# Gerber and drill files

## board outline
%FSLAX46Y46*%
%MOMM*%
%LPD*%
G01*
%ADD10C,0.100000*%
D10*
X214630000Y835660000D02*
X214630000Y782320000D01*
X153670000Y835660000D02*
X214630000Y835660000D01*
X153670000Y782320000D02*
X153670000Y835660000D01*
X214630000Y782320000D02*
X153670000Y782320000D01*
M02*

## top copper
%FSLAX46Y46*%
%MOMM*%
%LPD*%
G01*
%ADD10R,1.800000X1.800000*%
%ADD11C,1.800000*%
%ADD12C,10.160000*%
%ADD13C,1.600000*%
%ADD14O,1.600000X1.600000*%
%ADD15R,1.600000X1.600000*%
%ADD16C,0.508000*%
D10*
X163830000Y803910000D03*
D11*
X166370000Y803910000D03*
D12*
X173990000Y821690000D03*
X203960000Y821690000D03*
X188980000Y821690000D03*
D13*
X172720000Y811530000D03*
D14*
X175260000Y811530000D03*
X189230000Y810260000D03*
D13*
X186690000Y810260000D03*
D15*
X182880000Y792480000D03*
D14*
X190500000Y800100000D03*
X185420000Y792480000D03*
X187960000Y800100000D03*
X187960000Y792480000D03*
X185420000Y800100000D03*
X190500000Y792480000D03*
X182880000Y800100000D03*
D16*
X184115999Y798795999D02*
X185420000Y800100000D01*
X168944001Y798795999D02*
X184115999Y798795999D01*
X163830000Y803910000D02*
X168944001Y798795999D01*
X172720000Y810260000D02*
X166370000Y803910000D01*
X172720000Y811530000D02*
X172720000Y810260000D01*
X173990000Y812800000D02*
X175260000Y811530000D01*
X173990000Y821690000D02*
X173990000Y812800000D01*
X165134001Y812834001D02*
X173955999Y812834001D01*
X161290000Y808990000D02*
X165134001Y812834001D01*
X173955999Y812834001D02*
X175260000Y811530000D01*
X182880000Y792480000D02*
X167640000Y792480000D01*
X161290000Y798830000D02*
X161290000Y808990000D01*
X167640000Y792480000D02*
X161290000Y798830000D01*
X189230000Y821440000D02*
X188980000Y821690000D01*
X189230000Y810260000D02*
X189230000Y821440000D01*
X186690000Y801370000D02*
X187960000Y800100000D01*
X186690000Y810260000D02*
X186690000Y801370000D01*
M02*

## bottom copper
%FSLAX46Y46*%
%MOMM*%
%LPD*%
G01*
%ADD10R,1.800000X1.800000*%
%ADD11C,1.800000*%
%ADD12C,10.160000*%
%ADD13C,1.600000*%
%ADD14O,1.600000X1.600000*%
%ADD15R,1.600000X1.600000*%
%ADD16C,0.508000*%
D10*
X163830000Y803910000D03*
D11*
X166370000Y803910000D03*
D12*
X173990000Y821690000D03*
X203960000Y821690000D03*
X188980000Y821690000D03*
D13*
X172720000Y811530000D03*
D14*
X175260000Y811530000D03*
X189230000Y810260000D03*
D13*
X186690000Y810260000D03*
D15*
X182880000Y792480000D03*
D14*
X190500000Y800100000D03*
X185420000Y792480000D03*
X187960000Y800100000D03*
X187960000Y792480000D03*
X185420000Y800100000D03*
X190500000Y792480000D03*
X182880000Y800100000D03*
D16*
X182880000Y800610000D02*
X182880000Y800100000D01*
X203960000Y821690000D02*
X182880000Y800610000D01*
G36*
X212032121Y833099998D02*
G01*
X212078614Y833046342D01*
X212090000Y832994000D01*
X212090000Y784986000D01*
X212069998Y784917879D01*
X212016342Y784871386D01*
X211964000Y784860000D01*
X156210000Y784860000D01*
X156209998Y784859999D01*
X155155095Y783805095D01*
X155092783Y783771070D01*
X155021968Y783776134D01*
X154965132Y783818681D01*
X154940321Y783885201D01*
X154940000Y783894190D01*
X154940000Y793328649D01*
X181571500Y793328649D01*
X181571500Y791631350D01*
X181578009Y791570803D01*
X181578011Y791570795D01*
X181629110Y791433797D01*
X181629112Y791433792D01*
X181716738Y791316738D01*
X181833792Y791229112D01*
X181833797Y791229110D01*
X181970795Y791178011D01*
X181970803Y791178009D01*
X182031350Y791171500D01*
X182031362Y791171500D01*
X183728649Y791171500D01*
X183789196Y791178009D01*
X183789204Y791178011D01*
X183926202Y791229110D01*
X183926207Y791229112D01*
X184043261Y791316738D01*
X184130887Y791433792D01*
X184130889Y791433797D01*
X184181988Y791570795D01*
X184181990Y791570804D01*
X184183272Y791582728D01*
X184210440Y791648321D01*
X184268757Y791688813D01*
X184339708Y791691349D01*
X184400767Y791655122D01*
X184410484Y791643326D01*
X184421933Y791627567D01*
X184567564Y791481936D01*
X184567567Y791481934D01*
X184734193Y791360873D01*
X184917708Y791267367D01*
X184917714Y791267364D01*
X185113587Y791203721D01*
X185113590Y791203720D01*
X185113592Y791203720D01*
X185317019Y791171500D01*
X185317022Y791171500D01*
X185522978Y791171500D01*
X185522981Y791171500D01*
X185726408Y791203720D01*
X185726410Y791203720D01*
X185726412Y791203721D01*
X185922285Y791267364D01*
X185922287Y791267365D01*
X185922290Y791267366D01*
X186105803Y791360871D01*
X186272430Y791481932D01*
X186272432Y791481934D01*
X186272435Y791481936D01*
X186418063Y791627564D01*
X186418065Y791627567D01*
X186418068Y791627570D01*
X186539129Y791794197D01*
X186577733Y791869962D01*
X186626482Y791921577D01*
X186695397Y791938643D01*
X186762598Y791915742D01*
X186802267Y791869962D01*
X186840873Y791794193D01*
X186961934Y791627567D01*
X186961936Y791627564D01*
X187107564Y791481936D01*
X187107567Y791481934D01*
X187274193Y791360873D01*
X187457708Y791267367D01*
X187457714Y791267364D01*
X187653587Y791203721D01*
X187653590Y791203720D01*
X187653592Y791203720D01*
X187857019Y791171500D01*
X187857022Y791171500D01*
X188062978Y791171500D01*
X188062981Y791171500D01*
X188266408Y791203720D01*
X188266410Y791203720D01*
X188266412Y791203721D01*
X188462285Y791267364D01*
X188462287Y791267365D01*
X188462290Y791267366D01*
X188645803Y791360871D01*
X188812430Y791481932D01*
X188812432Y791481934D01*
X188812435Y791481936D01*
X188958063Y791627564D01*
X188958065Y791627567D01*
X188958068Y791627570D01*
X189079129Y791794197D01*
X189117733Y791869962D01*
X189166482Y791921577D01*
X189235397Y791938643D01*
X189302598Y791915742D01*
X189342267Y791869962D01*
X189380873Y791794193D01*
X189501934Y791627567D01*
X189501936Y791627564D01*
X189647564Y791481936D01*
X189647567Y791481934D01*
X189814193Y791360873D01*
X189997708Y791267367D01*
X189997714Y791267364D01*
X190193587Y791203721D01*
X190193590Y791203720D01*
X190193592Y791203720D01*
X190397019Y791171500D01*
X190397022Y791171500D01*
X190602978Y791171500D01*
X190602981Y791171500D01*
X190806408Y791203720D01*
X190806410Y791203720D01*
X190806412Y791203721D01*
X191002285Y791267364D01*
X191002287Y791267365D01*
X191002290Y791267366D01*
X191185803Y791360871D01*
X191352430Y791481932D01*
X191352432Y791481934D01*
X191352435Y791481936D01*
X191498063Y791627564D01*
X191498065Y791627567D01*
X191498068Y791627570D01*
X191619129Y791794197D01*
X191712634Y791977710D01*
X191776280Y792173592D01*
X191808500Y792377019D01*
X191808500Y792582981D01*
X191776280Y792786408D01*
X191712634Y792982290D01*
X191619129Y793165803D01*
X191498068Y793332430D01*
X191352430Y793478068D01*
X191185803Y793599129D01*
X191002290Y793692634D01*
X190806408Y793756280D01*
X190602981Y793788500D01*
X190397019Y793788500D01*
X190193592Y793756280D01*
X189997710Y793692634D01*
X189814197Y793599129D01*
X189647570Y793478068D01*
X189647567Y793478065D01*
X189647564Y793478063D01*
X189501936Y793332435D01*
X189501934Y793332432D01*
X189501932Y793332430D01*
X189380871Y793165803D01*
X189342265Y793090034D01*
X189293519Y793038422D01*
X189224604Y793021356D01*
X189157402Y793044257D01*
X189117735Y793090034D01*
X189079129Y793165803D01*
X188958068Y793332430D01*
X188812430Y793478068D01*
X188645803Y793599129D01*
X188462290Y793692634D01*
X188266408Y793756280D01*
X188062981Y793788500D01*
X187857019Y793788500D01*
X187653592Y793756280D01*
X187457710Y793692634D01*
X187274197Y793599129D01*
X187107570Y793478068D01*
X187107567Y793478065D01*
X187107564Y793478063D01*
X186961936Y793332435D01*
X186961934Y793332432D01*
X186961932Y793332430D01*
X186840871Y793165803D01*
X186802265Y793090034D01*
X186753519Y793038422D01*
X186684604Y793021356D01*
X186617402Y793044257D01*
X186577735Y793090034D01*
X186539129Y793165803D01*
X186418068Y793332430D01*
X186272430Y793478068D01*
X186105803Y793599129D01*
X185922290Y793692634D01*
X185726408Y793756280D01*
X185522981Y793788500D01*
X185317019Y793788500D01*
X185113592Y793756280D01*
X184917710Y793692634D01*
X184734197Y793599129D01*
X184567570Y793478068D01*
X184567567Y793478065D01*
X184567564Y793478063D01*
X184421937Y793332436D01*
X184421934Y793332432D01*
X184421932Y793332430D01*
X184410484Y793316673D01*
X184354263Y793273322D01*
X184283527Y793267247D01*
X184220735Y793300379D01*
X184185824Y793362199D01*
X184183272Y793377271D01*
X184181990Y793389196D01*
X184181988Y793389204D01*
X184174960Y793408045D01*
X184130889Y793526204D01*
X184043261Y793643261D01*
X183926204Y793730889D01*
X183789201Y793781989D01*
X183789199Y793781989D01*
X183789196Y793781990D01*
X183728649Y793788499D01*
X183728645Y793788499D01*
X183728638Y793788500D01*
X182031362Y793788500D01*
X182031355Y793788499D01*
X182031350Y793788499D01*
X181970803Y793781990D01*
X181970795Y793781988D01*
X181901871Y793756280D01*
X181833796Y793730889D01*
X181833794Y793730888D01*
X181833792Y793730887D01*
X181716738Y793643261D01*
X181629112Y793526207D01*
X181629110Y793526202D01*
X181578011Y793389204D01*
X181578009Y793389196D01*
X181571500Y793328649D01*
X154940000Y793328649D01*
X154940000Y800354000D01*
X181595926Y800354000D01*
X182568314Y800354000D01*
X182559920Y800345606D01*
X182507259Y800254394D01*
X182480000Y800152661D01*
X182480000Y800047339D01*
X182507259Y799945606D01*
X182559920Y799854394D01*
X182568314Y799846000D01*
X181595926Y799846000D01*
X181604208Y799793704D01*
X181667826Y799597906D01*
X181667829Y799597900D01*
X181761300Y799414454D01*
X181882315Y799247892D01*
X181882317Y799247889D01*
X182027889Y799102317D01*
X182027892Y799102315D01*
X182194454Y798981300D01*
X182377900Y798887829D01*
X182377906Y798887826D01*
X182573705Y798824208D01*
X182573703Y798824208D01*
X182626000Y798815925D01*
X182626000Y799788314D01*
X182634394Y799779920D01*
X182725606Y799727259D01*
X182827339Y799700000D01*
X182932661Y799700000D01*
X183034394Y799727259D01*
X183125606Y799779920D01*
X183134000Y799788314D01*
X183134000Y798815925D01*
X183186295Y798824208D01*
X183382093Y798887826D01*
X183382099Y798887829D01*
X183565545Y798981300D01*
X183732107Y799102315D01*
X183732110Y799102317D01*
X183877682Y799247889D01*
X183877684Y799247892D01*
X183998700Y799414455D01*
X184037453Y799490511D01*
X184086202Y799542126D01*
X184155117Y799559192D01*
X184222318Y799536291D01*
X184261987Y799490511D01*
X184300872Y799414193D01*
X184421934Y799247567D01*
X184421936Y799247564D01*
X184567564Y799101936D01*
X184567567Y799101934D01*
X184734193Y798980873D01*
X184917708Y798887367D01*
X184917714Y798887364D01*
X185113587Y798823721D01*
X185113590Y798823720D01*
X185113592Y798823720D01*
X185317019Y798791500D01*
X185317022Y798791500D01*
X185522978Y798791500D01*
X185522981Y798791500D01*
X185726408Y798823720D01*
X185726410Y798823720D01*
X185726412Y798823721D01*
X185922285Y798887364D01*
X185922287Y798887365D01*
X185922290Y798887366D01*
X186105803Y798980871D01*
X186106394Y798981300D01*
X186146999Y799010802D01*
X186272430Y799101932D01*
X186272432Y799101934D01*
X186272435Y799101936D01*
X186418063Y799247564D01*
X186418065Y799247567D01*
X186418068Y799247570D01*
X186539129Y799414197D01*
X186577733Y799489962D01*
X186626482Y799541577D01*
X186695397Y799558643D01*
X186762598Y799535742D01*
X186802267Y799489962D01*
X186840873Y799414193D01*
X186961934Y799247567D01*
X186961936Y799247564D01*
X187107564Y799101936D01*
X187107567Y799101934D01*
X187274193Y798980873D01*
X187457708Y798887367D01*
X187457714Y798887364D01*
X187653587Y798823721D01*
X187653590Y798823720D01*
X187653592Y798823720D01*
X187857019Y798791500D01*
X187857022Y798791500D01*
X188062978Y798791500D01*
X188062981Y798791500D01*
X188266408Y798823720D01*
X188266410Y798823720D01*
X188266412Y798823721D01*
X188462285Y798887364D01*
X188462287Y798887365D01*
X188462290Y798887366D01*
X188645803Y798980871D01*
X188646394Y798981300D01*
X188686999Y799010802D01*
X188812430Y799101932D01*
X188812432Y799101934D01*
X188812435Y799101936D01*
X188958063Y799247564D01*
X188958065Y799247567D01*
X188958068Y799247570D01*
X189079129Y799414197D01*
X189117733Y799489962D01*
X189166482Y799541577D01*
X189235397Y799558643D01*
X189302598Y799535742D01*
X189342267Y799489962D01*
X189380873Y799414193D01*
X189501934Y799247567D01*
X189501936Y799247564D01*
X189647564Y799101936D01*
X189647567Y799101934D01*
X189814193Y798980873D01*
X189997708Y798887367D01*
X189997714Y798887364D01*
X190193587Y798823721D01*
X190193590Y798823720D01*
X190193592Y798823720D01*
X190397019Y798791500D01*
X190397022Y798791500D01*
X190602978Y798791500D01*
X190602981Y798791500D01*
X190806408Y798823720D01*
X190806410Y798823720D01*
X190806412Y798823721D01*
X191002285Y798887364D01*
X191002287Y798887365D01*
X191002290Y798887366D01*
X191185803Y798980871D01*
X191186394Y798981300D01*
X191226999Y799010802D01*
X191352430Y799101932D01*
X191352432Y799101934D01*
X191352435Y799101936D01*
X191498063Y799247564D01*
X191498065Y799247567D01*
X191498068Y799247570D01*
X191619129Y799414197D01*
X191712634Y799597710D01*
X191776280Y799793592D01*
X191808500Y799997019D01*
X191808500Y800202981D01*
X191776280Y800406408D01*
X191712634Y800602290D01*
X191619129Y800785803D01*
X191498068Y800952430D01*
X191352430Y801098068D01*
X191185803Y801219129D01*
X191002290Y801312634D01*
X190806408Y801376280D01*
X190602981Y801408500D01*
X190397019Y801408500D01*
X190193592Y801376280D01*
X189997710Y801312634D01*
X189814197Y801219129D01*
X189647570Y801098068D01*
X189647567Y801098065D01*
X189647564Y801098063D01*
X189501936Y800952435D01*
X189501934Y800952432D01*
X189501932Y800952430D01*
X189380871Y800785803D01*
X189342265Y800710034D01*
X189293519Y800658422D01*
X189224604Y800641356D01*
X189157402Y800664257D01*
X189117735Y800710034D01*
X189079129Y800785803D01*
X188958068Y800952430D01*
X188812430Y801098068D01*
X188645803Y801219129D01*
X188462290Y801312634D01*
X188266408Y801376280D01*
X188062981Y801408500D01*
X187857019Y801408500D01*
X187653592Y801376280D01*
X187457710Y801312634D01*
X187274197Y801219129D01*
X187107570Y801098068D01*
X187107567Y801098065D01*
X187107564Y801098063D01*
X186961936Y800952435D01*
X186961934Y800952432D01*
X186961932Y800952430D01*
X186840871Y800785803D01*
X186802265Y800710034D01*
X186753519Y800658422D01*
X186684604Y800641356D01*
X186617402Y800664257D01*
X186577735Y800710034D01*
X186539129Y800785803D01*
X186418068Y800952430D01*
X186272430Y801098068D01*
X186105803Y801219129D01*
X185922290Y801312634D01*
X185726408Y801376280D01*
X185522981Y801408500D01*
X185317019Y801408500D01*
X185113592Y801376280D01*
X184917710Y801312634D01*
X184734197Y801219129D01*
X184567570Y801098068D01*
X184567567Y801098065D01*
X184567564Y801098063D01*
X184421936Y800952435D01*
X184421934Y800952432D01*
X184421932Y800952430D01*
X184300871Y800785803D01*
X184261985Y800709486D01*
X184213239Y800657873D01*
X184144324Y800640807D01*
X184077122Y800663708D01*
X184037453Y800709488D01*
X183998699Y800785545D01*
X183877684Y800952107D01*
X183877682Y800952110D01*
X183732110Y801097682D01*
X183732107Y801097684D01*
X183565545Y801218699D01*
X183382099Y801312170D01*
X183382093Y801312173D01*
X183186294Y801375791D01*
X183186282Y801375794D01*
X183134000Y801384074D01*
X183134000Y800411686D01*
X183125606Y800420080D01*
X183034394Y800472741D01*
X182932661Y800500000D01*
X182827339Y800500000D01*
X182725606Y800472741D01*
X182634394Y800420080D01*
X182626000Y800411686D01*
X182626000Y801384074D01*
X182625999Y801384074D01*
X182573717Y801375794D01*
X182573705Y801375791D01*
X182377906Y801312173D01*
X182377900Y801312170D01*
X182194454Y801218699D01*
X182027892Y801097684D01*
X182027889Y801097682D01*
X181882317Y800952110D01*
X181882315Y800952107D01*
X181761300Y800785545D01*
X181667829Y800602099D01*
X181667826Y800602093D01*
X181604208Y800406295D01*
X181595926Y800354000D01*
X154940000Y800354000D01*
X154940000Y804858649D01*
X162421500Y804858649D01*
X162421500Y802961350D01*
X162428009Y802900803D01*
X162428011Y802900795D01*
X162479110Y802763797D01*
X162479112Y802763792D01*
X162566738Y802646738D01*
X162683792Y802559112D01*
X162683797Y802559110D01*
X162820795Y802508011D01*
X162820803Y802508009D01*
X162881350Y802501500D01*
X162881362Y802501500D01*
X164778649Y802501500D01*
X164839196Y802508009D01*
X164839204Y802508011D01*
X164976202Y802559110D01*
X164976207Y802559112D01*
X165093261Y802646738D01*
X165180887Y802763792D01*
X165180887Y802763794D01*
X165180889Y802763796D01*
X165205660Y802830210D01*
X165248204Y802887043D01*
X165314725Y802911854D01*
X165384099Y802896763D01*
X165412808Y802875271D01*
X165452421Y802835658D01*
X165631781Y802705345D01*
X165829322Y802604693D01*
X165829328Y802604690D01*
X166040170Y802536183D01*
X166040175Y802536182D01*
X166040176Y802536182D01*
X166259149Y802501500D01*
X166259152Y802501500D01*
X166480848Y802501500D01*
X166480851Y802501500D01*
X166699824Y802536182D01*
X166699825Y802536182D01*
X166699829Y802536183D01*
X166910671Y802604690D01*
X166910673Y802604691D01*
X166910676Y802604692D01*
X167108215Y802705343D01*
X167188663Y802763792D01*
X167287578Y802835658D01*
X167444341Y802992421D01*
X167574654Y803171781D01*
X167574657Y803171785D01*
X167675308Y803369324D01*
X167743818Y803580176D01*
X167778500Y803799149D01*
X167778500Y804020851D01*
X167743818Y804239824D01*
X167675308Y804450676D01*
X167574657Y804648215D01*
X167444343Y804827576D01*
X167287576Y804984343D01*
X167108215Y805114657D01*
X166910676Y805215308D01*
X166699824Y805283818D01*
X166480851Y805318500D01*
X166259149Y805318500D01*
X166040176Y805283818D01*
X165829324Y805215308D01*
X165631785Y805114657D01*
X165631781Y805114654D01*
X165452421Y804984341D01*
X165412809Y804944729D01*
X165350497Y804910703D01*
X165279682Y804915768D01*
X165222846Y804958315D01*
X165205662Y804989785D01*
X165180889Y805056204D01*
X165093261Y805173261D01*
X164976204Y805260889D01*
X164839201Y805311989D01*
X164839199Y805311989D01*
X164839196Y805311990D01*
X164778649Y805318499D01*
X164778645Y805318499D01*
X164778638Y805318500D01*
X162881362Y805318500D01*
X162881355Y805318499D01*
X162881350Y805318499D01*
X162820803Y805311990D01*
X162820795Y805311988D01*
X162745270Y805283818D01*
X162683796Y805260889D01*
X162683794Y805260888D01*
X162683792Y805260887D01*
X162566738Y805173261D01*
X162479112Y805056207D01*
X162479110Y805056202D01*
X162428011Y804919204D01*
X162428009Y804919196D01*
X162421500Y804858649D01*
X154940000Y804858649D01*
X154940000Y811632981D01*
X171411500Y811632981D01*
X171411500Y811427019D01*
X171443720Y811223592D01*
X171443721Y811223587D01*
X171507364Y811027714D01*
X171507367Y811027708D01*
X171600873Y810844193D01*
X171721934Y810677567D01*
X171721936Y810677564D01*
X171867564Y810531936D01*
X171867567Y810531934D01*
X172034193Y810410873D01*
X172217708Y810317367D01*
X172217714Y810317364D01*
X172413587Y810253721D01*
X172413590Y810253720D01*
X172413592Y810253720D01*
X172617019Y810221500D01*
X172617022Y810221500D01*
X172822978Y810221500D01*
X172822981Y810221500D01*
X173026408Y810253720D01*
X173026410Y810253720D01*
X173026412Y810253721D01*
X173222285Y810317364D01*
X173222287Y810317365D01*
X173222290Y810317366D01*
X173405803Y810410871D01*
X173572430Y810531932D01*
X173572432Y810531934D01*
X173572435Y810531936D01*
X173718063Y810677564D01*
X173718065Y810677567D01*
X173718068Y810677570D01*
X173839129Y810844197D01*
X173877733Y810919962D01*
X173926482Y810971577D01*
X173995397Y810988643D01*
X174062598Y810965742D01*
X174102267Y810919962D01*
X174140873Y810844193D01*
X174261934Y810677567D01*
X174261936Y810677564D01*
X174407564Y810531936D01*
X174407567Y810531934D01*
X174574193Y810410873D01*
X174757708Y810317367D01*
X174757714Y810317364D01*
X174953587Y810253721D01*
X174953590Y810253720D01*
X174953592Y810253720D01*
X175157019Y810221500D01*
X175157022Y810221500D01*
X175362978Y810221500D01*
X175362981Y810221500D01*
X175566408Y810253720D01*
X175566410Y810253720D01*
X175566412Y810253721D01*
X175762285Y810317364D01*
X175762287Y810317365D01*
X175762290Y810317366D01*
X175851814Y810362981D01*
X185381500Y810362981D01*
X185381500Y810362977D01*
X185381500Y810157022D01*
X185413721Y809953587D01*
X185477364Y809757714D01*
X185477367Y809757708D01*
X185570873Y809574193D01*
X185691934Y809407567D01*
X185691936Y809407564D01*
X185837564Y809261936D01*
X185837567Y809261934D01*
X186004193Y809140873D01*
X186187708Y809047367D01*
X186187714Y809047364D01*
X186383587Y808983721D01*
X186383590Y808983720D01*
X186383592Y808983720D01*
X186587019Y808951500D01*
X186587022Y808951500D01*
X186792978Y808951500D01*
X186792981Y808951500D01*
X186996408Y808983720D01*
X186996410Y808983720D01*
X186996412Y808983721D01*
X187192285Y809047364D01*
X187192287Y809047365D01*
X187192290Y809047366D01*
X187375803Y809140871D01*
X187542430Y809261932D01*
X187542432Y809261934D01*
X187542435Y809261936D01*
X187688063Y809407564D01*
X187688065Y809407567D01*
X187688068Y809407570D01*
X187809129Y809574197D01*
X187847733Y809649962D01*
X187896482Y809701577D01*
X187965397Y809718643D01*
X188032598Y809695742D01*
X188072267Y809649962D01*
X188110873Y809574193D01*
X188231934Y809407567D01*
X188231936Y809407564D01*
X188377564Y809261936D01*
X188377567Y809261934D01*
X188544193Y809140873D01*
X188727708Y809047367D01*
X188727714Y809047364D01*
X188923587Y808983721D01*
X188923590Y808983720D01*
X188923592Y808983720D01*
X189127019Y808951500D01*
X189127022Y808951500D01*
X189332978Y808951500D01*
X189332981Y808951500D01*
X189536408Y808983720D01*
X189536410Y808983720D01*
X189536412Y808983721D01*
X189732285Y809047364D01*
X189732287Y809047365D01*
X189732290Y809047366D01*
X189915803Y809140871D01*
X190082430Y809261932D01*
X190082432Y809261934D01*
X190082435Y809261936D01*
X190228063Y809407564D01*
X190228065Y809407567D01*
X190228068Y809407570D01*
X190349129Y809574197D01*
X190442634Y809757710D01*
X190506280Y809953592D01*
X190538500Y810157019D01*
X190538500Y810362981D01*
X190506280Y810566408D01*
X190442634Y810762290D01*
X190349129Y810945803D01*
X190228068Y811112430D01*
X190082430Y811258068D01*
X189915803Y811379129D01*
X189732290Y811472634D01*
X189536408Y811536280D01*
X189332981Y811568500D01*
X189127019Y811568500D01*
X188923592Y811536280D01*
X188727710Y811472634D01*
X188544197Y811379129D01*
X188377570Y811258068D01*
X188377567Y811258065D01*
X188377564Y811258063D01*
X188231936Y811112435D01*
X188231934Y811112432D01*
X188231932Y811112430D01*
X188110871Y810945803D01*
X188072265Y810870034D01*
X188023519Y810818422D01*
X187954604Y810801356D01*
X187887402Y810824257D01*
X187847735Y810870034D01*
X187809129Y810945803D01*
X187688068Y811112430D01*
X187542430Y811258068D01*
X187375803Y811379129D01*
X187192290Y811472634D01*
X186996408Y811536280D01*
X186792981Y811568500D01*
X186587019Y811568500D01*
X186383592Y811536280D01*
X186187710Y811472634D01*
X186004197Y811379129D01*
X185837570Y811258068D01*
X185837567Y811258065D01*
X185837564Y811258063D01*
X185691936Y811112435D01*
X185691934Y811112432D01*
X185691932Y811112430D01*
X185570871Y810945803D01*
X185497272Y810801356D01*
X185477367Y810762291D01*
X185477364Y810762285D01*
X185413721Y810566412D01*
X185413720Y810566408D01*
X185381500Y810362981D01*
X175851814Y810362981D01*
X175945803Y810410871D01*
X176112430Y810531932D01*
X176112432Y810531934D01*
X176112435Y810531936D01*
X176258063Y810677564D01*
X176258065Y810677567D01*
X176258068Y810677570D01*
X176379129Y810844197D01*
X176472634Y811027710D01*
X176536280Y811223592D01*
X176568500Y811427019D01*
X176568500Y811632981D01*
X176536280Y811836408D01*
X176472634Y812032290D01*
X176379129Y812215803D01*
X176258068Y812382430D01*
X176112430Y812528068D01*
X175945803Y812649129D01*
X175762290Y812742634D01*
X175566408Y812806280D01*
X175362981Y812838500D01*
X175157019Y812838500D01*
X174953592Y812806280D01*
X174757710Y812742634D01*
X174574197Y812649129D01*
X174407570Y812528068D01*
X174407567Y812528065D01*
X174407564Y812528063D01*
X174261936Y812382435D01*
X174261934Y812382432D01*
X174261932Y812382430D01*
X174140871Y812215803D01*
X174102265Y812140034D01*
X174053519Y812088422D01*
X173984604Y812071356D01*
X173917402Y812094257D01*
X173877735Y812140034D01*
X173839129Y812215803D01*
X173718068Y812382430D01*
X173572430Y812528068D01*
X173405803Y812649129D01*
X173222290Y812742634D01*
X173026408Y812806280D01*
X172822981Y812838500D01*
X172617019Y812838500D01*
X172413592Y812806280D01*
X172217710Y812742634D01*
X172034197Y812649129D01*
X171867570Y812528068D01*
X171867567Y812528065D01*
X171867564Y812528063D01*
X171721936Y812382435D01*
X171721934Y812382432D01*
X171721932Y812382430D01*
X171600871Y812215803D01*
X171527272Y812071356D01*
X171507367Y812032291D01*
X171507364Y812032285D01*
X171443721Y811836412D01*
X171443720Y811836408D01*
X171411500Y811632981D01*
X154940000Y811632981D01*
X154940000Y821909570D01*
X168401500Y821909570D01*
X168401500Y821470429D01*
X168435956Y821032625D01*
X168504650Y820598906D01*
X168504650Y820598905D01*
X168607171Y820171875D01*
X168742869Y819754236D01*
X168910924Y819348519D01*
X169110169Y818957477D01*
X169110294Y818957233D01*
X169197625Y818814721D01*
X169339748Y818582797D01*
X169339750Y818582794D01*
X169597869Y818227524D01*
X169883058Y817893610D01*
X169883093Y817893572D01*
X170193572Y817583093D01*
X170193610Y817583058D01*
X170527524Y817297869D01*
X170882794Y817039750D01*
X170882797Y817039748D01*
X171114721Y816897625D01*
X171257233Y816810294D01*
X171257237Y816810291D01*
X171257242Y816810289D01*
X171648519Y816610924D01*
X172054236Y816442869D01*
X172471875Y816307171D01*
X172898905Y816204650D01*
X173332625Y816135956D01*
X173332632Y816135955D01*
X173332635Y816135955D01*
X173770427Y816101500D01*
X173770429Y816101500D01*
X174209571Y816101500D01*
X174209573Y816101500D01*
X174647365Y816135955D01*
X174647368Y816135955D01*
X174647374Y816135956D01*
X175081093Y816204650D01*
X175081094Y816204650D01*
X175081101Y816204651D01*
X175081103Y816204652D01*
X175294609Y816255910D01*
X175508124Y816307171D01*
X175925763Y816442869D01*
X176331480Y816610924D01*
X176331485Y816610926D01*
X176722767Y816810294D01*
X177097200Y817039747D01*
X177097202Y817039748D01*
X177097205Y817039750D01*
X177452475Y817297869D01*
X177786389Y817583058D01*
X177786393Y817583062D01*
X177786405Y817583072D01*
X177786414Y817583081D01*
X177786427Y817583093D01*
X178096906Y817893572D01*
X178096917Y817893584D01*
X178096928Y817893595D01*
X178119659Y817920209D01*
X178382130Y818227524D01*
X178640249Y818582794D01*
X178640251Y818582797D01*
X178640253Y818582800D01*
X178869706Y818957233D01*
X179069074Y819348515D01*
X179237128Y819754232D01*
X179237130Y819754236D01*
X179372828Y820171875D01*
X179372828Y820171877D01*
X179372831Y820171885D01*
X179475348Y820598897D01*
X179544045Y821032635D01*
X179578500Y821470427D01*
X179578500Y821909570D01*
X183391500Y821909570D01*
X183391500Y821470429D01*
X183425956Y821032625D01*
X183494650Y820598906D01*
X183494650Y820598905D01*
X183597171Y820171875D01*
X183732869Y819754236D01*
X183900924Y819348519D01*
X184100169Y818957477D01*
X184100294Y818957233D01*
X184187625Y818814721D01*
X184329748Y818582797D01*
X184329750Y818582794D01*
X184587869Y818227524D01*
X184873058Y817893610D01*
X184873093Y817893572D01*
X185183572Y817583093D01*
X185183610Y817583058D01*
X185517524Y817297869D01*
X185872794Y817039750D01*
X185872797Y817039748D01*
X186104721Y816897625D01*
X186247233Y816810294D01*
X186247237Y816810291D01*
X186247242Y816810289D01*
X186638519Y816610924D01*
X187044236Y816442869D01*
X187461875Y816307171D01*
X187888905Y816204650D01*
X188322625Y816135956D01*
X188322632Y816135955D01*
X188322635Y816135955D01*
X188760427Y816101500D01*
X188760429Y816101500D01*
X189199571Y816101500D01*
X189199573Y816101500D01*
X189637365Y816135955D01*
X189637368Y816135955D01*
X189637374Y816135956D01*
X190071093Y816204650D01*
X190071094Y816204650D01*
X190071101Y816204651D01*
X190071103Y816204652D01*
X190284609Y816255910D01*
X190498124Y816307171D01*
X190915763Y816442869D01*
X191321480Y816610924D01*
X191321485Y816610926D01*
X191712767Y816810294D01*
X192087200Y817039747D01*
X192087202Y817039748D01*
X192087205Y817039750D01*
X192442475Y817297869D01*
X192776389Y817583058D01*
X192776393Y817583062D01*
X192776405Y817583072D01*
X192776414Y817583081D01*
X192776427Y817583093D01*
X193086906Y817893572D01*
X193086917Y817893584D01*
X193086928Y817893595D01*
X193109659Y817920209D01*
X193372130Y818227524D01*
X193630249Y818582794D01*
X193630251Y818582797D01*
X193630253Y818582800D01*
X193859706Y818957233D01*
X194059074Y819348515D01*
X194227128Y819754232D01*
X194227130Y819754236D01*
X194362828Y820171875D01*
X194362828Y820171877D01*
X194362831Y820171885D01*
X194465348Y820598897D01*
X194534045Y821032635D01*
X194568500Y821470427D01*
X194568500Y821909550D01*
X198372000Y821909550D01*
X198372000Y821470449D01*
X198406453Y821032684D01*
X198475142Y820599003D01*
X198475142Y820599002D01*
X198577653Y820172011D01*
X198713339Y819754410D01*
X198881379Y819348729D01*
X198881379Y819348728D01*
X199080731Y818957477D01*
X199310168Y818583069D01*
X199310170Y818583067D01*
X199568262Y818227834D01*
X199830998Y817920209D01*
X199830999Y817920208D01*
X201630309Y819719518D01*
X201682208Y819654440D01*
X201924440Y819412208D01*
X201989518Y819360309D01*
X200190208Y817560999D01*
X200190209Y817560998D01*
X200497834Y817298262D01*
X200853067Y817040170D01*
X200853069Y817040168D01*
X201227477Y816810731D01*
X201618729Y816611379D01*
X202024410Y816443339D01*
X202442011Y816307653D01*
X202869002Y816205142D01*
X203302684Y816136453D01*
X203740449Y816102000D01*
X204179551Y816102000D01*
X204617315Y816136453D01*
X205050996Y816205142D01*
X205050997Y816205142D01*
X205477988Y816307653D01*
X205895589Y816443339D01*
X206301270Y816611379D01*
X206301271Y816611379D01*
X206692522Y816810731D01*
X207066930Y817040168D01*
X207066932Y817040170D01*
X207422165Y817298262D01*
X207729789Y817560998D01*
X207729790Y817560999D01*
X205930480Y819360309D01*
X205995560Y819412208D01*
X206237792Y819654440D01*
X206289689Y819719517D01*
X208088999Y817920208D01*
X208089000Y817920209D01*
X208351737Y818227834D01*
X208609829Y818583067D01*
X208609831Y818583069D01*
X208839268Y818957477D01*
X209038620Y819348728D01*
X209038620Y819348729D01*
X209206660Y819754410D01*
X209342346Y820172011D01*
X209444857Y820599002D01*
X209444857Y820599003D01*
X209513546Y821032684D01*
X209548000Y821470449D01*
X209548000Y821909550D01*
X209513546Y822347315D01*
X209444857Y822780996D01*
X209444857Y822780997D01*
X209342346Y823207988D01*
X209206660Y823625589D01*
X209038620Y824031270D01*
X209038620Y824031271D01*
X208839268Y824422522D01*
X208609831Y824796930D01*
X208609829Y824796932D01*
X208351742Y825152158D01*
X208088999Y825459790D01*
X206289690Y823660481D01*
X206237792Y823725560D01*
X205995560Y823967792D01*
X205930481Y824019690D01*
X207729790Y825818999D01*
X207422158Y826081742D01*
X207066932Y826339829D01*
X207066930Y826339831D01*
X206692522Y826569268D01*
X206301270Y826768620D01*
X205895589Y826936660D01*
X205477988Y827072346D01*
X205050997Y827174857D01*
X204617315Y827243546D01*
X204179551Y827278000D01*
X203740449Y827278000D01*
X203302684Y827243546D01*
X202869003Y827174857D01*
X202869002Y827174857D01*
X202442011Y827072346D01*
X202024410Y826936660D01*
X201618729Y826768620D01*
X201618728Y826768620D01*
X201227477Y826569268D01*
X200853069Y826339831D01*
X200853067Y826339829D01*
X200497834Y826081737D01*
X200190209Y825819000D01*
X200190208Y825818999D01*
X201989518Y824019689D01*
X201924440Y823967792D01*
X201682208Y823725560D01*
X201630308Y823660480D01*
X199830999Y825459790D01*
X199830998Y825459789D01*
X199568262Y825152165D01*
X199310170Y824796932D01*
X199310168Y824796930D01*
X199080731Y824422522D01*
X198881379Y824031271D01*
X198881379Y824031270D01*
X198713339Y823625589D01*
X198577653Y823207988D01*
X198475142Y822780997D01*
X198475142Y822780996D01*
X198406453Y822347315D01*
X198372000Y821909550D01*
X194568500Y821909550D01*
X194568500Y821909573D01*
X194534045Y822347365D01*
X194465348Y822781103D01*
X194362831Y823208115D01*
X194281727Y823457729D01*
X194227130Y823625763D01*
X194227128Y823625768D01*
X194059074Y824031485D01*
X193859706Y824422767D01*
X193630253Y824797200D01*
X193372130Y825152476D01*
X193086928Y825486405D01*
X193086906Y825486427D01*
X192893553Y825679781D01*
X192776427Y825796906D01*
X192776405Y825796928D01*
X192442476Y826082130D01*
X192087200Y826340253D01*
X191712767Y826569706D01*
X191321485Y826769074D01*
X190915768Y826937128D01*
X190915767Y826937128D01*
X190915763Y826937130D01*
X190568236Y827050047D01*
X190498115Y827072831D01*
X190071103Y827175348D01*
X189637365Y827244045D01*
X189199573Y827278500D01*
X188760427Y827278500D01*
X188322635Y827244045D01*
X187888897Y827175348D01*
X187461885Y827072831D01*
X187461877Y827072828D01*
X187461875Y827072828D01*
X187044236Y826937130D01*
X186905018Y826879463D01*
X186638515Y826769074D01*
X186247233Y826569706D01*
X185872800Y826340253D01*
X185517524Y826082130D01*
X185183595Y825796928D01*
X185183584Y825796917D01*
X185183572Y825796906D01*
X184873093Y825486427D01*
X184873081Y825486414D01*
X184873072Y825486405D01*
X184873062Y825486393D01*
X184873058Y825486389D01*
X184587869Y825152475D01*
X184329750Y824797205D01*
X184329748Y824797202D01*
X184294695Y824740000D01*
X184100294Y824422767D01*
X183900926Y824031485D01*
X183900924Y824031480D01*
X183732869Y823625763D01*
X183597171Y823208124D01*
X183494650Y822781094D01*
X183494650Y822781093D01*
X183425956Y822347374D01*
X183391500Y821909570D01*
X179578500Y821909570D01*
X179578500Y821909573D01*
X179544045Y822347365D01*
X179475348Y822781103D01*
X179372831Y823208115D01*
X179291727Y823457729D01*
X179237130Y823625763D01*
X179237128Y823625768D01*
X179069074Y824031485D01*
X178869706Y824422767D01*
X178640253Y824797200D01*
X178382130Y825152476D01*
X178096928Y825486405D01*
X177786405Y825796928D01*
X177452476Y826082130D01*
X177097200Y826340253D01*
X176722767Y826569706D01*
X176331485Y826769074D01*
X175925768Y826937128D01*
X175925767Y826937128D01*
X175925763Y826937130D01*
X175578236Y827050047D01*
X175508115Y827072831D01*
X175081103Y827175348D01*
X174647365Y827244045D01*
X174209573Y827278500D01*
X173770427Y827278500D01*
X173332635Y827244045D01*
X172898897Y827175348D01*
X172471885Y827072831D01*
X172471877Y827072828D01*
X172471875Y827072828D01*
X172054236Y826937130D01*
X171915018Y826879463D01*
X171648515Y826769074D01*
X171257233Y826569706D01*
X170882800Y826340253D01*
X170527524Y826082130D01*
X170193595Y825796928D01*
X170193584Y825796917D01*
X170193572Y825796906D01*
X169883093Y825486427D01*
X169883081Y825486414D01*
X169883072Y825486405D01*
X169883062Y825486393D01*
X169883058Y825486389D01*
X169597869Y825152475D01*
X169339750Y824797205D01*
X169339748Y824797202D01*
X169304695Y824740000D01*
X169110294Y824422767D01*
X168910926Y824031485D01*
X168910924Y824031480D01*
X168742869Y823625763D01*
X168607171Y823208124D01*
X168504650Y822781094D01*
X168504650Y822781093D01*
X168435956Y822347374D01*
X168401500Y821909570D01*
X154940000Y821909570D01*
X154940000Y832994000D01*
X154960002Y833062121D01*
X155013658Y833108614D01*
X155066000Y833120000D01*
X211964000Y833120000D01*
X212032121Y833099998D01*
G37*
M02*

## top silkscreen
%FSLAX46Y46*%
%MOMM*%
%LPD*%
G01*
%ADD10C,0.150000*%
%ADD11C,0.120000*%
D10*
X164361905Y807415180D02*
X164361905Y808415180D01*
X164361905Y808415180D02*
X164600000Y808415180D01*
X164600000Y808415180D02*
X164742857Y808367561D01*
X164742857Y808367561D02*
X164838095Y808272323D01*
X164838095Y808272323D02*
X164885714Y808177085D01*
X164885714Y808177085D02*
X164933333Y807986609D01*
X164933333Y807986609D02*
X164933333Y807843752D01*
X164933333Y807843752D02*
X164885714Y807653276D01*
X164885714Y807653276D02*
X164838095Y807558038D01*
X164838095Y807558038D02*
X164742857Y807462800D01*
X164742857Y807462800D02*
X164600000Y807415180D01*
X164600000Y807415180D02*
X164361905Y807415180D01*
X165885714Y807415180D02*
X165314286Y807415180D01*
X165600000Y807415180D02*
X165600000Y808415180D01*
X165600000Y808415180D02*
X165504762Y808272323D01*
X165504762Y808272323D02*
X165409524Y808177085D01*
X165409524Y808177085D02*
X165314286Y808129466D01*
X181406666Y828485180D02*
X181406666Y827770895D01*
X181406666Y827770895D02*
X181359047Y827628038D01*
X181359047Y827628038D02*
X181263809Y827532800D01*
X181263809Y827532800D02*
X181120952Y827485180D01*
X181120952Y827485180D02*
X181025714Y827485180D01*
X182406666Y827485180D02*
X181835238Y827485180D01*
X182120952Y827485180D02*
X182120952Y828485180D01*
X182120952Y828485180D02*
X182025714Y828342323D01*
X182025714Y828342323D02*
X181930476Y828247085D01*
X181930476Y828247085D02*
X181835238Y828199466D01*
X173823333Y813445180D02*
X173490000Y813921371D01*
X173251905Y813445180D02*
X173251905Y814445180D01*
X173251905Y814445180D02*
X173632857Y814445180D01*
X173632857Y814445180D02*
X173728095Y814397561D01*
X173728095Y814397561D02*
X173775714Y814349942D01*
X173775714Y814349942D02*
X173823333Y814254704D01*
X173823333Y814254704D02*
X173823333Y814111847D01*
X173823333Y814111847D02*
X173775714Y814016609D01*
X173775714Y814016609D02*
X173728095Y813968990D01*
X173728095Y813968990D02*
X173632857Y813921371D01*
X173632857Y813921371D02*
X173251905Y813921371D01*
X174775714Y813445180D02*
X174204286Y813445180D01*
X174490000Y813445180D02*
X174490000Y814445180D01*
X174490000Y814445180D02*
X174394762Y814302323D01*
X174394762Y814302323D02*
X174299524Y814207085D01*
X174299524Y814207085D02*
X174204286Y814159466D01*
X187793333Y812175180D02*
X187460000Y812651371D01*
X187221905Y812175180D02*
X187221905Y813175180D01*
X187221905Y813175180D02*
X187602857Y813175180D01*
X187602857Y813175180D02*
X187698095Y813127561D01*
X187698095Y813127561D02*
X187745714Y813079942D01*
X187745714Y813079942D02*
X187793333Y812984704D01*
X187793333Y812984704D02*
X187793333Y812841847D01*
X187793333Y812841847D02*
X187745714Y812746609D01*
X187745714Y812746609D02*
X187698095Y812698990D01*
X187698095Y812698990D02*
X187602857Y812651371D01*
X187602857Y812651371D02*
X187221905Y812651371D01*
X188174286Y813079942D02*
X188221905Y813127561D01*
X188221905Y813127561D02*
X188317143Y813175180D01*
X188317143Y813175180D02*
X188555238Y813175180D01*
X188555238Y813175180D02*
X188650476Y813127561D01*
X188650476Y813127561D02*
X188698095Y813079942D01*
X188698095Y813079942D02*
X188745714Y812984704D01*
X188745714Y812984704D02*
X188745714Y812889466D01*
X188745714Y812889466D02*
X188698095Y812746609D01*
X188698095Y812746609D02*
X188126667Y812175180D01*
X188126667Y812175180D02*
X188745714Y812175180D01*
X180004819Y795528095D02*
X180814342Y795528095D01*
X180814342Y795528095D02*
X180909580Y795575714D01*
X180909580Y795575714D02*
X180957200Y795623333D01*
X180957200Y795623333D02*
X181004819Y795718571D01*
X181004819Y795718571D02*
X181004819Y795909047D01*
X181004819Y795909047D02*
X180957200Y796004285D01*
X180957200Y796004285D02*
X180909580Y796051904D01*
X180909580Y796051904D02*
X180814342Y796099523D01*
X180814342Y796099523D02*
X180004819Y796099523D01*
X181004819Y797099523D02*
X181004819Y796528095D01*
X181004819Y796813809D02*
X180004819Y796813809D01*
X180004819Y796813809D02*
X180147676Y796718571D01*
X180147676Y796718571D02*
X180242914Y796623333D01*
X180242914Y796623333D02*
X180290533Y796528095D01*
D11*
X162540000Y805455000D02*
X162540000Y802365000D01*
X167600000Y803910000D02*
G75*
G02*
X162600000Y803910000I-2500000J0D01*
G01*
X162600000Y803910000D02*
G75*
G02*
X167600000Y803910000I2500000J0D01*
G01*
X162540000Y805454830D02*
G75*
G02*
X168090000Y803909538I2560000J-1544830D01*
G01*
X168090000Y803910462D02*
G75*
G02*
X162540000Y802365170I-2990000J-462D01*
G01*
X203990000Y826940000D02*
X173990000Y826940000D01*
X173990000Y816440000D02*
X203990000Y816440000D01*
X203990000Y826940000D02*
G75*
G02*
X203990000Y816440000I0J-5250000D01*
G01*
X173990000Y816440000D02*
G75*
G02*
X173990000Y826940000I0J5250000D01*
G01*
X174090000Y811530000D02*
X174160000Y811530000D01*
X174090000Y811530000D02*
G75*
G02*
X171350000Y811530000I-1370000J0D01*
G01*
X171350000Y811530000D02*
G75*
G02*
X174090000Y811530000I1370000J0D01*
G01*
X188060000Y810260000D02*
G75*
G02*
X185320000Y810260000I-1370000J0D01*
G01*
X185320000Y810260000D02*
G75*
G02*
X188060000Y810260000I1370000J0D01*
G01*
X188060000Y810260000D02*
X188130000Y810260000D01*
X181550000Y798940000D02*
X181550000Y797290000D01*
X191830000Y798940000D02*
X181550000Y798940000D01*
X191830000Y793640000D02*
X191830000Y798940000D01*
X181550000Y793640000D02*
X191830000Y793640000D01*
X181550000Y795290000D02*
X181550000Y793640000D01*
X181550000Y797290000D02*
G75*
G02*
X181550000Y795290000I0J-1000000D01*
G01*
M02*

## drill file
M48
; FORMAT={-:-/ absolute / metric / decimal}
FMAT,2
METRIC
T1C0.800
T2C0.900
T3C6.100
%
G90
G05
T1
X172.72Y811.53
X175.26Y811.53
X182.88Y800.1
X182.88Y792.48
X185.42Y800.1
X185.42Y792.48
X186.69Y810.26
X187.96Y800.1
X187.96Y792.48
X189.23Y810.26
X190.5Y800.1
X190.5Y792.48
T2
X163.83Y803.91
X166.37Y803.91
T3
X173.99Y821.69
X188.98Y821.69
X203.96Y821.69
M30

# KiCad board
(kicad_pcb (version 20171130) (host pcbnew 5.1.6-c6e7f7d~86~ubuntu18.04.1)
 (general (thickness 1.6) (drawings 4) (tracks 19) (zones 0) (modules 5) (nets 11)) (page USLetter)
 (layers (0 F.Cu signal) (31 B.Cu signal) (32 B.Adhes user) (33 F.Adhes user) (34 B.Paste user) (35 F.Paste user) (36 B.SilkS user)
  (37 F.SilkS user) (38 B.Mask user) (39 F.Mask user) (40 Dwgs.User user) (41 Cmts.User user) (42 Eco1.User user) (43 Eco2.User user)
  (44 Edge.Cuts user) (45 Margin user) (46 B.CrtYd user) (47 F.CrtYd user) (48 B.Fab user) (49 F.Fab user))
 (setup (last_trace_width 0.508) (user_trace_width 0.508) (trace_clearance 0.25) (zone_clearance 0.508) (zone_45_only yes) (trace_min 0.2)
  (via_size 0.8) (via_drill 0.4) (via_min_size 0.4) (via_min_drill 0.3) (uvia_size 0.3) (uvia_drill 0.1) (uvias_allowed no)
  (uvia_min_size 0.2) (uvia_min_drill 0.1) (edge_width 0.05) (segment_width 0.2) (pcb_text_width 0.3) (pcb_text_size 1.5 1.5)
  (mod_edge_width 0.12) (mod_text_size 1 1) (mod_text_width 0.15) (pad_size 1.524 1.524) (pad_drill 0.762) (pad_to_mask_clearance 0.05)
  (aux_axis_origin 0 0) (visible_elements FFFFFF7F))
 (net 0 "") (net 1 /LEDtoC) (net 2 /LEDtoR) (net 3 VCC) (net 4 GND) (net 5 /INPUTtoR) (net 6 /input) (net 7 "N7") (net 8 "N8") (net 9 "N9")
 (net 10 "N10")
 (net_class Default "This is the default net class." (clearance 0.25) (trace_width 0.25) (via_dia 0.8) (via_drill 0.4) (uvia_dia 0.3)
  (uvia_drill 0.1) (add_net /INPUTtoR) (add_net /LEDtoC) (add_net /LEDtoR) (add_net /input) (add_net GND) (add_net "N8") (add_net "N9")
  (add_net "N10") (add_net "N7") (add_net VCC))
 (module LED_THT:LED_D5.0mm (layer F.Cu) (at 163.83 -803.91)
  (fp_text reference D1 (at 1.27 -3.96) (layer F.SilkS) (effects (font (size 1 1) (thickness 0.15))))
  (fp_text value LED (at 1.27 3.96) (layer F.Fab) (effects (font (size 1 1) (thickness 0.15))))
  (fp_line (start -1.29 -1.545) (end -1.29 1.545) (layer F.SilkS) (width 0.12))
  (fp_circle (center 1.27 0) (end 3.77 0) (layer F.SilkS) (width 0.12))
  (fp_arc (start 1.27 0) (end -1.29 -1.54483) (angle 148.9) (layer F.SilkS) (width 0.12))
  (fp_arc (start 1.27 0) (end -1.29 1.54483) (angle -148.9) (layer F.SilkS) (width 0.12))
  (pad 1 thru_hole rect (at 0 0) (size 1.8 1.8) (drill 0.9) (layers *.Cu *.Mask) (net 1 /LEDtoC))
  (pad 2 thru_hole circle (at 2.54 0) (size 1.8 1.8) (drill 0.9) (layers *.Cu *.Mask) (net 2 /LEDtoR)))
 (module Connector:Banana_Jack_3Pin (layer F.Cu) (at 173.99 -821.69)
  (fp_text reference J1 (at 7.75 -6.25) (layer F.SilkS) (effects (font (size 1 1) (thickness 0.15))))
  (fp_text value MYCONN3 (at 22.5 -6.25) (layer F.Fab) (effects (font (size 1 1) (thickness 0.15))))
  (fp_line (start 30 -5.25) (end 0 -5.25) (layer F.SilkS) (width 0.12))
  (fp_line (start 0 5.25) (end 30 5.25) (layer F.SilkS) (width 0.12))
  (fp_arc (start 30 0) (end 30 -5.25) (angle 180) (layer F.SilkS) (width 0.12))
  (fp_arc (start 0 0) (end 0 5.25) (angle 180) (layer F.SilkS) (width 0.12))
  (pad 1 thru_hole circle (at 0 0) (size 10.16 10.16) (drill 6.1) (layers *.Cu *.Mask) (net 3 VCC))
  (pad 3 thru_hole circle (at 29.97 0) (size 10.16 10.16) (drill 6.1) (layers *.Cu *.Mask) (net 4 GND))
  (pad 2 thru_hole circle (at 14.99 0) (size 10.16 10.16) (drill 6.1) (layers *.Cu *.Mask) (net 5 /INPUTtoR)))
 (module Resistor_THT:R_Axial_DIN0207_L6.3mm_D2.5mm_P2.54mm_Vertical (layer F.Cu) (at 172.72 -811.53)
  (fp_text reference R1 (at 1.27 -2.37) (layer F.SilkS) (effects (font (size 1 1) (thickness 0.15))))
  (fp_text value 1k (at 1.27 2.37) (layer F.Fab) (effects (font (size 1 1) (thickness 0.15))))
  (fp_line (start 1.37 0) (end 1.44 0) (layer F.SilkS) (width 0.12))
  (fp_circle (center 0 0) (end 1.37 0) (layer F.SilkS) (width 0.12))
  (pad 1 thru_hole circle (at 0 0) (size 1.6 1.6) (drill 0.8) (layers *.Cu *.Mask) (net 2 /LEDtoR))
  (pad 2 thru_hole oval (at 2.54 0) (size 1.6 1.6) (drill 0.8) (layers *.Cu *.Mask) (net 3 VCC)))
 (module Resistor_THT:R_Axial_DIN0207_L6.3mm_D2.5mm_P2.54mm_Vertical (layer F.Cu) (at 186.69 -810.26)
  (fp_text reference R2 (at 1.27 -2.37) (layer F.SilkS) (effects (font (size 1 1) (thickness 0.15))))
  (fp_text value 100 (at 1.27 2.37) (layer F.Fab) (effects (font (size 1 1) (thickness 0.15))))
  (fp_circle (center 0 0) (end 1.37 0) (layer F.SilkS) (width 0.12))
  (fp_line (start 1.37 0) (end 1.44 0) (layer F.SilkS) (width 0.12))
  (pad 2 thru_hole oval (at 2.54 0) (size 1.6 1.6) (drill 0.8) (layers *.Cu *.Mask) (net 5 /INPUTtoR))
  (pad 1 thru_hole circle (at 0 0) (size 1.6 1.6) (drill 0.8) (layers *.Cu *.Mask) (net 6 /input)))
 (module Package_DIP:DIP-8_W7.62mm (layer F.Cu) (at 182.88 -792.48 90)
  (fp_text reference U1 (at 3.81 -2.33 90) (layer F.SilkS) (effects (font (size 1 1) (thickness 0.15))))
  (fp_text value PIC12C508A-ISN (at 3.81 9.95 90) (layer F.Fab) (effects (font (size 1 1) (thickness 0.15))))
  (fp_line (start 6.46 -1.33) (end 4.81 -1.33) (layer F.SilkS) (width 0.12))
  (fp_line (start 6.46 8.95) (end 6.46 -1.33) (layer F.SilkS) (width 0.12))
  (fp_line (start 1.16 8.95) (end 6.46 8.95) (layer F.SilkS) (width 0.12))
  (fp_line (start 1.16 -1.33) (end 1.16 8.95) (layer F.SilkS) (width 0.12))
  (fp_line (start 2.81 -1.33) (end 1.16 -1.33) (layer F.SilkS) (width 0.12))
  (fp_arc (start 3.81 -1.33) (end 2.81 -1.33) (angle -180) (layer F.SilkS) (width 0.12))
  (pad 1 thru_hole rect (at 0 0 90) (size 1.6 1.6) (drill 0.8) (layers *.Cu *.Mask) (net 3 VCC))
  (pad 5 thru_hole oval (at 7.62 7.62 90) (size 1.6 1.6) (drill 0.8) (layers *.Cu *.Mask) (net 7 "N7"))
  (pad 2 thru_hole oval (at 0 2.54 90) (size 1.6 1.6) (drill 0.8) (layers *.Cu *.Mask) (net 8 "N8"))
  (pad 6 thru_hole oval (at 7.62 5.08 90) (size 1.6 1.6) (drill 0.8) (layers *.Cu *.Mask) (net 6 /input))
  (pad 3 thru_hole oval (at 0 5.08 90) (size 1.6 1.6) (drill 0.8) (layers *.Cu *.Mask) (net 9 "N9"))
  (pad 7 thru_hole oval (at 7.62 2.54 90) (size 1.6 1.6) (drill 0.8) (layers *.Cu *.Mask) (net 1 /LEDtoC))
  (pad 4 thru_hole oval (at 0 7.62 90) (size 1.6 1.6) (drill 0.8) (layers *.Cu *.Mask) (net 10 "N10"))
  (pad 8 thru_hole oval (at 7.62 0 90) (size 1.6 1.6) (drill 0.8) (layers *.Cu *.Mask) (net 4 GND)))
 (gr_line (start 214.63 -835.66) (end 214.63 -782.32) (layer Edge.Cuts) (width 0.1))
 (gr_line (start 153.67 -835.66) (end 214.63 -835.66) (layer Edge.Cuts) (width 0.1))
 (gr_line (start 153.67 -782.32) (end 153.67 -835.66) (layer Edge.Cuts) (width 0.1))
 (gr_line (start 214.63 -782.32) (end 153.67 -782.32) (layer Edge.Cuts) (width 0.1))
 (segment (start 184.115999 -798.795999) (end 185.42 -800.1) (width 0.508) (layer F.Cu) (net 1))
 (segment (start 168.944001 -798.795999) (end 184.115999 -798.795999) (width 0.508) (layer F.Cu) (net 1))
 (segment (start 163.83 -803.91) (end 168.944001 -798.795999) (width 0.508) (layer F.Cu) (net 1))
 (segment (start 172.72 -810.26) (end 166.37 -803.91) (width 0.508) (layer F.Cu) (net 2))
 (segment (start 172.72 -811.53) (end 172.72 -810.26) (width 0.508) (layer F.Cu) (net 2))
 (segment (start 173.99 -812.8) (end 175.26 -811.53) (width 0.508) (layer F.Cu) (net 3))
 (segment (start 173.99 -821.69) (end 173.99 -812.8) (width 0.508) (layer F.Cu) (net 3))
 (segment (start 165.134001 -812.834001) (end 173.955999 -812.834001) (width 0.508) (layer F.Cu) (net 3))
 (segment (start 161.29 -808.99) (end 165.134001 -812.834001) (width 0.508) (layer F.Cu) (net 3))
 (segment (start 173.955999 -812.834001) (end 175.26 -811.53) (width 0.508) (layer F.Cu) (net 3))
 (segment (start 182.88 -792.48) (end 167.64 -792.48) (width 0.508) (layer F.Cu) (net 3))
 (segment (start 161.29 -798.83) (end 161.29 -808.99) (width 0.508) (layer F.Cu) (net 3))
 (segment (start 167.64 -792.48) (end 161.29 -798.83) (width 0.508) (layer F.Cu) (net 3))
 (segment (start 182.88 -800.61) (end 182.88 -800.1) (width 0.508) (layer B.Cu) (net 4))
 (segment (start 203.96 -821.69) (end 182.88 -800.61) (width 0.508) (layer B.Cu) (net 4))
 (segment (start 189.23 -821.44) (end 188.98 -821.69) (width 0.508) (layer F.Cu) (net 5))
 (segment (start 189.23 -810.26) (end 189.23 -821.44) (width 0.508) (layer F.Cu) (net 5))
 (segment (start 186.69 -801.37) (end 187.96 -800.1) (width 0.508) (layer F.Cu) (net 6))
 (segment (start 186.69 -810.26) (end 186.69 -801.37) (width 0.508) (layer F.Cu) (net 6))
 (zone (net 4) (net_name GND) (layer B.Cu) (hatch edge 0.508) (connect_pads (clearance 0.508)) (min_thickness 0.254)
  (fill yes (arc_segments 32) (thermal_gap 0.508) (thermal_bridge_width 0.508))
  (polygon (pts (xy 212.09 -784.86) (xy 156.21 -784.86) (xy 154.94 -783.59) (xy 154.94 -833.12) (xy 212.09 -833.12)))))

